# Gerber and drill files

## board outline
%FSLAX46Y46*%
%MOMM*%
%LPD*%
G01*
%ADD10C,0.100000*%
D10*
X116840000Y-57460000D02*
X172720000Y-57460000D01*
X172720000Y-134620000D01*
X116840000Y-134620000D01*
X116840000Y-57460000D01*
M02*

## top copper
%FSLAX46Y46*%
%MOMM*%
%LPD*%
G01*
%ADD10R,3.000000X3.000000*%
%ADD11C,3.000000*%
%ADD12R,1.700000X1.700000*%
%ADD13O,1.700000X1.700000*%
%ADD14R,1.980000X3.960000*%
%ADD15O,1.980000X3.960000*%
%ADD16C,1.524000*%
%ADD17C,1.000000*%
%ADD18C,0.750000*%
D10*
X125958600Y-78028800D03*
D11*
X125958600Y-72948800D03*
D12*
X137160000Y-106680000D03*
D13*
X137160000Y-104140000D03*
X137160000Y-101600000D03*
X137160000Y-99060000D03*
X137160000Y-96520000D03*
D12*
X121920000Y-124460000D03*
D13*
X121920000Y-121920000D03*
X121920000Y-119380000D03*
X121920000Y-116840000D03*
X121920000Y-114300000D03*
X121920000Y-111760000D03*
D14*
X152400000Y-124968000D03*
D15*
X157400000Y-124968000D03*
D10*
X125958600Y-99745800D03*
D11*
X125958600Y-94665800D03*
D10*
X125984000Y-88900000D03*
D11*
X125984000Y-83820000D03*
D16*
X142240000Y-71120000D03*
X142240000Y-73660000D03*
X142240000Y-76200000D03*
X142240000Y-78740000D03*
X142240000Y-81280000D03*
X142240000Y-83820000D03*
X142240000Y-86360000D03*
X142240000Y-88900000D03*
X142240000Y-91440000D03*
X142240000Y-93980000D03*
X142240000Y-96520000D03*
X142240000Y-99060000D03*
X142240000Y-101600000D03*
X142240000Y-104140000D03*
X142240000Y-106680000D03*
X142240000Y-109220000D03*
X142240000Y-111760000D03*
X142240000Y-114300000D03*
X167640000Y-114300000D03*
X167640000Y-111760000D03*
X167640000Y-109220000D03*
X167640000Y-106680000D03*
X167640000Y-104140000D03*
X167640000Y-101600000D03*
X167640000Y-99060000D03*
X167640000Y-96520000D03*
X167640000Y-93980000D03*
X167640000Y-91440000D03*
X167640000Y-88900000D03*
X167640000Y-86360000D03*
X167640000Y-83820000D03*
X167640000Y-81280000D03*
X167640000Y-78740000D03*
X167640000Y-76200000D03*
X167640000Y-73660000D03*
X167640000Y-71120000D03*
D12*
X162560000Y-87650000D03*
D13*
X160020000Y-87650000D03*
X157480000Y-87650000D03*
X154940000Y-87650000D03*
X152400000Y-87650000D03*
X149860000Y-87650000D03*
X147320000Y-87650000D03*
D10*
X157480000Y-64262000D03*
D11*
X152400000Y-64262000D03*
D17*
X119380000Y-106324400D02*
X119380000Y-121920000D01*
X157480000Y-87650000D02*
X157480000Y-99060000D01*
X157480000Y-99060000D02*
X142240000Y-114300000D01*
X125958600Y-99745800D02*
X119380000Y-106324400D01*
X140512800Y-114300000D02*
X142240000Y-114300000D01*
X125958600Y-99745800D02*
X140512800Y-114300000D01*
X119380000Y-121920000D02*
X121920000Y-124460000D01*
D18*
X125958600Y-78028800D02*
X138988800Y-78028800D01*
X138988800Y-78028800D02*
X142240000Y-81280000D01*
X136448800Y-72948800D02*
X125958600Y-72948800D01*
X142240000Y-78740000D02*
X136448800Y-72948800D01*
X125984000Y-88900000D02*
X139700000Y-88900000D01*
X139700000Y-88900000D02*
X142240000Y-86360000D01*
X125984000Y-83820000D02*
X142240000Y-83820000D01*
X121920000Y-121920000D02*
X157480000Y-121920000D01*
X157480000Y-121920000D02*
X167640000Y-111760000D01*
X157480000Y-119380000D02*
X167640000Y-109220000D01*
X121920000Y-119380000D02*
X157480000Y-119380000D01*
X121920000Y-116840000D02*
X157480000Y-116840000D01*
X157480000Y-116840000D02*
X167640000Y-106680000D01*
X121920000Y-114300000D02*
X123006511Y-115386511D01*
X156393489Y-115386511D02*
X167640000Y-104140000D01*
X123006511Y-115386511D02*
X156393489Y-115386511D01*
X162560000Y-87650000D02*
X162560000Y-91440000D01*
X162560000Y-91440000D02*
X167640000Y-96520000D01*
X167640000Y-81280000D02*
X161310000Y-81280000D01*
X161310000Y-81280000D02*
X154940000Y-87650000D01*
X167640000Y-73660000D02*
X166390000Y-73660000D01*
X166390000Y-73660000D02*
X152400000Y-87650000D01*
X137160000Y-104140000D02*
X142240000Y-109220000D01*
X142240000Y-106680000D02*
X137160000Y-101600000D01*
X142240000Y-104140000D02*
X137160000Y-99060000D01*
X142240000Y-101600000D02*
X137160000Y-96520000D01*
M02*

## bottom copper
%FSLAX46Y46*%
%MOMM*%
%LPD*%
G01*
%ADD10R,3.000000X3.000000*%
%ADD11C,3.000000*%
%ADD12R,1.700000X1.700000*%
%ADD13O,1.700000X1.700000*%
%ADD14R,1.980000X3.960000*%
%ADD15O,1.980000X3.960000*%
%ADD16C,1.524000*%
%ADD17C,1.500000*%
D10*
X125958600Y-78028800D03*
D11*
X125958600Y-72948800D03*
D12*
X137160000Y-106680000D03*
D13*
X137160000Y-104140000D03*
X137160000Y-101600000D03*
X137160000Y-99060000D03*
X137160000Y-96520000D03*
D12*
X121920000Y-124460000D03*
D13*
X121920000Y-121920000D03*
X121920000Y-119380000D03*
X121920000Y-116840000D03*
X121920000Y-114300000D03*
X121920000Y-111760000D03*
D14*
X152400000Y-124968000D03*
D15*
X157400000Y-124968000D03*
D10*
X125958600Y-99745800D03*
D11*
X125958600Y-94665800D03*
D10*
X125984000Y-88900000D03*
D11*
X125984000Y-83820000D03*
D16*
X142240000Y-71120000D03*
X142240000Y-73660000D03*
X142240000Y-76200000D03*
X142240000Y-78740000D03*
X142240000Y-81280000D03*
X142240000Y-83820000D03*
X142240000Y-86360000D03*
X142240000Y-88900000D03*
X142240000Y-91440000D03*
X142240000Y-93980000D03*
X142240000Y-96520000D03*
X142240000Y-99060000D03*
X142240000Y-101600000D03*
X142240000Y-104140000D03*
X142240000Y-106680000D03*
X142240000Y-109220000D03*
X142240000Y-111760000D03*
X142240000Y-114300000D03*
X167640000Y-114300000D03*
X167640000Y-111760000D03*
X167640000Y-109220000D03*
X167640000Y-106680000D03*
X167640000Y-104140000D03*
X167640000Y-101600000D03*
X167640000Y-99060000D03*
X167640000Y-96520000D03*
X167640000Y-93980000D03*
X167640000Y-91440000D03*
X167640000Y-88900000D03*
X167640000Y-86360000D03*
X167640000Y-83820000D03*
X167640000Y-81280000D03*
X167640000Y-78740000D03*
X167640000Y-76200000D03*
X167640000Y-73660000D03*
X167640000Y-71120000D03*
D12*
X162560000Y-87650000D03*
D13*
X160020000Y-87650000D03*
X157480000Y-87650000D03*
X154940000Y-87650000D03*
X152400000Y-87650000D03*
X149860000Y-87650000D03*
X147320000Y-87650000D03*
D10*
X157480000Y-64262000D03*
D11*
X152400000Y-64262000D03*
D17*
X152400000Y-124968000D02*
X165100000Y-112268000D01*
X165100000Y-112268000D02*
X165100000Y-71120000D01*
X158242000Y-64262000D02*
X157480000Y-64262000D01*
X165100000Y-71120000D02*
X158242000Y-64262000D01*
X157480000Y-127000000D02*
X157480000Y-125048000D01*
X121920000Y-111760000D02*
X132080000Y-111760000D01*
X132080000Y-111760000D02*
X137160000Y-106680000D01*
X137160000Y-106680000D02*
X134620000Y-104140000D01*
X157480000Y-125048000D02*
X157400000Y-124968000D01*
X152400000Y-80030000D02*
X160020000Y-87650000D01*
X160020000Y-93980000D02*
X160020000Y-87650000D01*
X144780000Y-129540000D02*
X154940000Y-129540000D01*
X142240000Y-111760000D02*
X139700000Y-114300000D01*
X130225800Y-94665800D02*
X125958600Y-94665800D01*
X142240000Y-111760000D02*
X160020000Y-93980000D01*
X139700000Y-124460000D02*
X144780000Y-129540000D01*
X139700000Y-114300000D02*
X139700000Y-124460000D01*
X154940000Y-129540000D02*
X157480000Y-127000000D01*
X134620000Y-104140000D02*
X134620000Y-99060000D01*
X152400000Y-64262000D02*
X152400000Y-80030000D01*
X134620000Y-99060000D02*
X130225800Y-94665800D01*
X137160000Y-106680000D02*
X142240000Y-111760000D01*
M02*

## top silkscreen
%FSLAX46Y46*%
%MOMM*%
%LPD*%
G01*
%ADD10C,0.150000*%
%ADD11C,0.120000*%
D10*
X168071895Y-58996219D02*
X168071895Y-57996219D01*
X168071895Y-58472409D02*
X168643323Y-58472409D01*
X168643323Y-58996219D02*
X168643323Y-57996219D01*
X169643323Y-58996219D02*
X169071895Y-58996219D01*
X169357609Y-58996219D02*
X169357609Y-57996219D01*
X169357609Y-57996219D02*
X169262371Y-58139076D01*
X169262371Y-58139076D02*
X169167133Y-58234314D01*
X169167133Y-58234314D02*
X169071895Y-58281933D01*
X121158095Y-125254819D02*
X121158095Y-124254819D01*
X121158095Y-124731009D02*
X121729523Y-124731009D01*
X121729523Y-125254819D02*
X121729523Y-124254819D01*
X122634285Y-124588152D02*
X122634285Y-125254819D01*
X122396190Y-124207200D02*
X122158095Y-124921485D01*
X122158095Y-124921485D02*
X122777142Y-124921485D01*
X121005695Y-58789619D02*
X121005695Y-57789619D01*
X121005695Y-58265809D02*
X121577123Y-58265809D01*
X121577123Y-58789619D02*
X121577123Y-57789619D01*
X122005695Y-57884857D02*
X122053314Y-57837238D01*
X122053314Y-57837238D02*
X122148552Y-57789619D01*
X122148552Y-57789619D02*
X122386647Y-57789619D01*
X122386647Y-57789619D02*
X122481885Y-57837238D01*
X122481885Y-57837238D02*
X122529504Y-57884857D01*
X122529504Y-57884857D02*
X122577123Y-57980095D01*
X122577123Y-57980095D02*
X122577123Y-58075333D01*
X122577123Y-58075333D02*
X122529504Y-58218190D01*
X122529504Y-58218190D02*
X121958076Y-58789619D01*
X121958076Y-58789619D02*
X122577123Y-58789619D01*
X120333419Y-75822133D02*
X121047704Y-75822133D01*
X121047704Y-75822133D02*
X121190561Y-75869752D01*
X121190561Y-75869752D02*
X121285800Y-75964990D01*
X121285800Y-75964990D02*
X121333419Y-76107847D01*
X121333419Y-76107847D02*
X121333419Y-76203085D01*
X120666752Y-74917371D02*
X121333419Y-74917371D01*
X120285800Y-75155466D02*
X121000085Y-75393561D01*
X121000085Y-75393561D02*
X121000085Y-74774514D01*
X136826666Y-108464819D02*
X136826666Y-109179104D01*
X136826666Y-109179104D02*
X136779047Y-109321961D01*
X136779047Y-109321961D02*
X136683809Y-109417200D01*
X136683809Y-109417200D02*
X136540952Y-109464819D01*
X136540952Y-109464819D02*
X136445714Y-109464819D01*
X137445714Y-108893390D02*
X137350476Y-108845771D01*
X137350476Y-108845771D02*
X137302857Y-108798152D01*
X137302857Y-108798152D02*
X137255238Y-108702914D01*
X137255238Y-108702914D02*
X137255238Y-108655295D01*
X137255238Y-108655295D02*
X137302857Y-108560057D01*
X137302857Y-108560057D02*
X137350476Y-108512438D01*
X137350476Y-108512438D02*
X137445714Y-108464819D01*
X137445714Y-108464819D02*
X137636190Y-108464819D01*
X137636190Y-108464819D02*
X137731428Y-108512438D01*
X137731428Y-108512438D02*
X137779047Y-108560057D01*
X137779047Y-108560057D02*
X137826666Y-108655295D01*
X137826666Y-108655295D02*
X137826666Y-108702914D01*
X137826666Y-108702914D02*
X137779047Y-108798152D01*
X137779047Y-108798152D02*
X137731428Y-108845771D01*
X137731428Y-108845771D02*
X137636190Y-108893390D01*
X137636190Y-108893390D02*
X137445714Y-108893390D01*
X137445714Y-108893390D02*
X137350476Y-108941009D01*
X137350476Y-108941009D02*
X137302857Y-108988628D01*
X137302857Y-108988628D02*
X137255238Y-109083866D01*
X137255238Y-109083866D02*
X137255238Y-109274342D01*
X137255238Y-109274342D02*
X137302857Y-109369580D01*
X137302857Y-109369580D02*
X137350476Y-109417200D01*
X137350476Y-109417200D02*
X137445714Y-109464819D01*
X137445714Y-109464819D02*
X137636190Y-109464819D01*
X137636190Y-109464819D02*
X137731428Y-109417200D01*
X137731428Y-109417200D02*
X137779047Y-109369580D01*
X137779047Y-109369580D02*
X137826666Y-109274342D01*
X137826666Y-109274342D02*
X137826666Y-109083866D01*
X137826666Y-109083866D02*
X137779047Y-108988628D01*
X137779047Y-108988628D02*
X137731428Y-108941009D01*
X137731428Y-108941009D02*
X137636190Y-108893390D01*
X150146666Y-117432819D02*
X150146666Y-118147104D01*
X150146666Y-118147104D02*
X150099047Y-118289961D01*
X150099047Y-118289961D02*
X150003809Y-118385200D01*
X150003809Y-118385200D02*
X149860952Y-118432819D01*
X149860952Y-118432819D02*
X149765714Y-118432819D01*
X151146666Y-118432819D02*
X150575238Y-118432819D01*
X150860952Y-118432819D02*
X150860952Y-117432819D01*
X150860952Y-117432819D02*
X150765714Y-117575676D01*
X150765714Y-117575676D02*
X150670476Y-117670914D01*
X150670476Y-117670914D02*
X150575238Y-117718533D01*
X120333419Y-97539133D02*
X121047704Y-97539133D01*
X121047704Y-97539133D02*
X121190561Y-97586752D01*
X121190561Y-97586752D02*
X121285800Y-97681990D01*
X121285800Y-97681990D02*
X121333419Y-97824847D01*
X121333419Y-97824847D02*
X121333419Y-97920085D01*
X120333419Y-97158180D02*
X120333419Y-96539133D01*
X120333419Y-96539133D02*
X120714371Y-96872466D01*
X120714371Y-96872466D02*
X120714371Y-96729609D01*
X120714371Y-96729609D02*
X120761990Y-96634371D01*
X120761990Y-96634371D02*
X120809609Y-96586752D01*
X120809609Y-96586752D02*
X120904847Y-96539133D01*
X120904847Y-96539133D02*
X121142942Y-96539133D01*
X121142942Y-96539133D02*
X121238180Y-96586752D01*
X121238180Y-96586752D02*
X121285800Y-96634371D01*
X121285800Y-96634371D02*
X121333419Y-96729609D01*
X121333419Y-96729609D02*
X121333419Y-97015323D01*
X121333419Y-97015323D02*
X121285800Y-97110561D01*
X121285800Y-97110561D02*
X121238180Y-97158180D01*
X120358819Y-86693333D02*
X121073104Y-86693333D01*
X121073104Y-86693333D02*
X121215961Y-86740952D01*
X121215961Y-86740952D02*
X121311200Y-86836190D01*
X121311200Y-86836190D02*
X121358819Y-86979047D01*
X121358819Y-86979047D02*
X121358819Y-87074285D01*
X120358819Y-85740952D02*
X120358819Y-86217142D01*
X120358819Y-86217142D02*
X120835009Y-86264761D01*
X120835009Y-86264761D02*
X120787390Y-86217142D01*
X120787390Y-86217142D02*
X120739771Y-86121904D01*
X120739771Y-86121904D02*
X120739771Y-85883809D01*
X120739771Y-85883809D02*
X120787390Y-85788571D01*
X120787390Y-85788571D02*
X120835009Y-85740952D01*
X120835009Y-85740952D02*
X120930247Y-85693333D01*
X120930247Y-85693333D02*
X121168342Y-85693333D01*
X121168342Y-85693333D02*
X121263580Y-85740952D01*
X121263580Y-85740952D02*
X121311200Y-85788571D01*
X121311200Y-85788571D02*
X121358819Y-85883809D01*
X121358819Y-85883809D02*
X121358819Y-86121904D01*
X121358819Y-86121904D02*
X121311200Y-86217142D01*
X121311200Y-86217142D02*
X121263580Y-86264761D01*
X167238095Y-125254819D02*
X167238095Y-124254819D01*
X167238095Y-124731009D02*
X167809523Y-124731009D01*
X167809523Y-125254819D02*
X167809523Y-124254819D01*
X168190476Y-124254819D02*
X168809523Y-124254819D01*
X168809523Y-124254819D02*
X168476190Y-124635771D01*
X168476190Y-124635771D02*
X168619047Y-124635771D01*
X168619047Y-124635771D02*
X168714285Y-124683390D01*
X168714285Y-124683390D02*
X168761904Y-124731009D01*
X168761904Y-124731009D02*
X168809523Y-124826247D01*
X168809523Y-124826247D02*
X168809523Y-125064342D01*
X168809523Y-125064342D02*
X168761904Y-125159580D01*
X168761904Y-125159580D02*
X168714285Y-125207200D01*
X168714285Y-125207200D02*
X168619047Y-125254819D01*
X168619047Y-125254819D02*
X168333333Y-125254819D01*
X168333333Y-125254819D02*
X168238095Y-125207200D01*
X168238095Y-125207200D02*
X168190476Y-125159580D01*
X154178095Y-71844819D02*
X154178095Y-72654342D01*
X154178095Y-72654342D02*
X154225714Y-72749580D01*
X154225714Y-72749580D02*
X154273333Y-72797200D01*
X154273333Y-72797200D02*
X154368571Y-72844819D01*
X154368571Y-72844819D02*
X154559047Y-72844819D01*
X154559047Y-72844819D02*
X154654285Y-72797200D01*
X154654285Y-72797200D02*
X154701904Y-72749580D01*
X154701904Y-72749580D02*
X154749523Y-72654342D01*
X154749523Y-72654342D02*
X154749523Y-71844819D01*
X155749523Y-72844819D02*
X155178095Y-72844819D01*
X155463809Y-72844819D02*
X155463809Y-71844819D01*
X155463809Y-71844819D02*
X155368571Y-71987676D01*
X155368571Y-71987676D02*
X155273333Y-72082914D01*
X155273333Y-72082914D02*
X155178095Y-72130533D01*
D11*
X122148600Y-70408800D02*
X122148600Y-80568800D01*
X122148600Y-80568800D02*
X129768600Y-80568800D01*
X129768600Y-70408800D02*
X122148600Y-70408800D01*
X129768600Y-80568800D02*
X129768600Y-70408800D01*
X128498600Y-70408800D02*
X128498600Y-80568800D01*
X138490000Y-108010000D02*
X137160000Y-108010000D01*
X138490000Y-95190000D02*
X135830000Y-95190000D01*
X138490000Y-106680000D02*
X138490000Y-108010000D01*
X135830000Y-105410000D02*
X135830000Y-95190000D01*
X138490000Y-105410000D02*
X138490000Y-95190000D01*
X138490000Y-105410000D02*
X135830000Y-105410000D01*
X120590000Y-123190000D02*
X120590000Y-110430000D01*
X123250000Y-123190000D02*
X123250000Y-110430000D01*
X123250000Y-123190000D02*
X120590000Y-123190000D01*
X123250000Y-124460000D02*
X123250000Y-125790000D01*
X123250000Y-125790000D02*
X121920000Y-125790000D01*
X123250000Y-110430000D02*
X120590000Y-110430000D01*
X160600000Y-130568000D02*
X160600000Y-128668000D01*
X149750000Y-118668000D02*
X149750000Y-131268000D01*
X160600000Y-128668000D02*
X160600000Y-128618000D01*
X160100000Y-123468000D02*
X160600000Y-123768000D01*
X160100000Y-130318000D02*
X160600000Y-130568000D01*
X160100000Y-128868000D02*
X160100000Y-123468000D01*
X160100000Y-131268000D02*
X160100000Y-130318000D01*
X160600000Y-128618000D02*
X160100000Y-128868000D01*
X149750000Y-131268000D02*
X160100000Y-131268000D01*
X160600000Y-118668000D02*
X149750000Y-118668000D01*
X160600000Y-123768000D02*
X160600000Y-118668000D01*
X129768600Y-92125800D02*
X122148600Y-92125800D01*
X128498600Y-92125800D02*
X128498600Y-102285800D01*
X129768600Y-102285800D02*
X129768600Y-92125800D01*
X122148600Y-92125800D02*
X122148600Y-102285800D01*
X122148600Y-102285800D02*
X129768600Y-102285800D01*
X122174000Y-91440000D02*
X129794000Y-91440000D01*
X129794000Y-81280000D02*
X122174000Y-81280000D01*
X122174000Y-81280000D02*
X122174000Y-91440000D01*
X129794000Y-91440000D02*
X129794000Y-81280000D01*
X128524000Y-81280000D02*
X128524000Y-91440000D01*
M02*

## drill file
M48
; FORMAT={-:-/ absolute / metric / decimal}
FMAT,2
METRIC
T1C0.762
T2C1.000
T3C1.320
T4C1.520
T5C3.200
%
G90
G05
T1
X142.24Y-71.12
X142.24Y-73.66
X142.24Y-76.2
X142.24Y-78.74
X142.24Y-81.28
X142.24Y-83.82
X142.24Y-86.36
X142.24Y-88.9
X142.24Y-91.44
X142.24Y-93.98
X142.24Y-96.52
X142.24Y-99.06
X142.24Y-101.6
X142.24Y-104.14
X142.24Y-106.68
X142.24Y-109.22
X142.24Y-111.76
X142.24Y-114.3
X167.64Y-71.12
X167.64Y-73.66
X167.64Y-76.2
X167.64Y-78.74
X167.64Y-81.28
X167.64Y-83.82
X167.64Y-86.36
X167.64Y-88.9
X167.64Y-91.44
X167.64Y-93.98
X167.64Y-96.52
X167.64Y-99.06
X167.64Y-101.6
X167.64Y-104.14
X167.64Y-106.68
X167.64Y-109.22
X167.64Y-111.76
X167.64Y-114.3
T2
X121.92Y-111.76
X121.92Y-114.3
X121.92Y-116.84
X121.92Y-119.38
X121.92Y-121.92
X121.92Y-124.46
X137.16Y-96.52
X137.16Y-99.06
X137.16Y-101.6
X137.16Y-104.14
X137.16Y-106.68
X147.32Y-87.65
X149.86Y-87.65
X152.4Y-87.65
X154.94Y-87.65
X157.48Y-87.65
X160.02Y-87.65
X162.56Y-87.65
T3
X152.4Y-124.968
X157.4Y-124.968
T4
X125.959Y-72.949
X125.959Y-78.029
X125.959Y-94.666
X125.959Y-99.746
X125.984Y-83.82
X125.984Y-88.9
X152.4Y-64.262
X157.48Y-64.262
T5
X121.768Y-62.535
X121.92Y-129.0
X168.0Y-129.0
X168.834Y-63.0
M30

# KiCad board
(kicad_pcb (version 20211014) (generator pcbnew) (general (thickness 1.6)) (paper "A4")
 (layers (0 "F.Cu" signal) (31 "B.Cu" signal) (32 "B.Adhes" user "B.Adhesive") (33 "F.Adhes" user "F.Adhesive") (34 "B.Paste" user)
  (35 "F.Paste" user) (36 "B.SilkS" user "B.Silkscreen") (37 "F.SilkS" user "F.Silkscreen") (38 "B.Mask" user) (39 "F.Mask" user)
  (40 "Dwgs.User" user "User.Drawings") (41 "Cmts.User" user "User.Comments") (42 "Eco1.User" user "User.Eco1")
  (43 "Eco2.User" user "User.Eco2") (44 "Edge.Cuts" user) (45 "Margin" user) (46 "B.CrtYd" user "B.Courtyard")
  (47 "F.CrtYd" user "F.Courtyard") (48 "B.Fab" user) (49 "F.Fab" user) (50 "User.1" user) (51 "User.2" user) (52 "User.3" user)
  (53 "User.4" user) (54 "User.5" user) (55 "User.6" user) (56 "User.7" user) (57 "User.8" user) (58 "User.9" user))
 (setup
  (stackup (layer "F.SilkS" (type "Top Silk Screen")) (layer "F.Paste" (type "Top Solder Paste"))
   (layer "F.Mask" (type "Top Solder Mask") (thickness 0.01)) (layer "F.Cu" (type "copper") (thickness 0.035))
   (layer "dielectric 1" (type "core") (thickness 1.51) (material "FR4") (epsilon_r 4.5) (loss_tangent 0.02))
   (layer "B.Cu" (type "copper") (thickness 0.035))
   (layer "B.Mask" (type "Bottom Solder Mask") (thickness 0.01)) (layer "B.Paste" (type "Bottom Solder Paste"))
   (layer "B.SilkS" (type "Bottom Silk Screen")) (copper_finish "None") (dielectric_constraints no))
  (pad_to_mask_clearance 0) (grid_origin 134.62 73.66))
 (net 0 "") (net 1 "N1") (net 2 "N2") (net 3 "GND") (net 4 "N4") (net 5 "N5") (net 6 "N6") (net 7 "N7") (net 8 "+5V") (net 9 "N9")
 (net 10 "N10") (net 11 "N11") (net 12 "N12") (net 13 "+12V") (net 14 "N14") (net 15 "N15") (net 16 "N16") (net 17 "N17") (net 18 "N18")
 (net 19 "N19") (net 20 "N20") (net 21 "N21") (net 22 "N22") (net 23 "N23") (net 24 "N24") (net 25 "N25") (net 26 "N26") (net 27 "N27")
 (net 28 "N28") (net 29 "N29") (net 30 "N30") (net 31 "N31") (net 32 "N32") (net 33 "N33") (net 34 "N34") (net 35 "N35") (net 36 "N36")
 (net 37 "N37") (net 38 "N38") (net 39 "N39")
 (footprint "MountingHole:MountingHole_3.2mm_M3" (layer "F.Cu") (at 168.8338 63)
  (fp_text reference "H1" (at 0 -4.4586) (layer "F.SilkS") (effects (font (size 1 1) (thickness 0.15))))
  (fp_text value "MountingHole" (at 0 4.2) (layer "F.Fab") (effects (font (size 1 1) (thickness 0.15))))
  (pad "" np_thru_hole circle (at 0 0) (size 3.2 3.2) (drill 3.2) (layers *.Cu *.Mask)))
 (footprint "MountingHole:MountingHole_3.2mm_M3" (layer "F.Cu") (at 121.92 129)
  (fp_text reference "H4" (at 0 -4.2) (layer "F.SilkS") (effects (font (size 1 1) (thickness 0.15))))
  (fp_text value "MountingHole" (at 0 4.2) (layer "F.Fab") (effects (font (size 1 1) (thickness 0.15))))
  (pad "" np_thru_hole circle (at 0 0) (size 3.2 3.2) (drill 3.2) (layers *.Cu *.Mask)))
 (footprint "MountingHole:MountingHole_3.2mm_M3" (layer "F.Cu") (at 121.7676 62.5348)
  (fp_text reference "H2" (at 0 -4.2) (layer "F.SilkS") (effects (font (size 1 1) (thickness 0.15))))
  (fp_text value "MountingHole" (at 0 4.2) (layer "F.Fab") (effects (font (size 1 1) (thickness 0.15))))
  (pad "" np_thru_hole circle (at 0 0) (size 3.2 3.2) (drill 3.2) (layers *.Cu *.Mask)))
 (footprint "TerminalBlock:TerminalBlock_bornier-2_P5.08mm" (layer "F.Cu") (at 125.9586 78.0288 90)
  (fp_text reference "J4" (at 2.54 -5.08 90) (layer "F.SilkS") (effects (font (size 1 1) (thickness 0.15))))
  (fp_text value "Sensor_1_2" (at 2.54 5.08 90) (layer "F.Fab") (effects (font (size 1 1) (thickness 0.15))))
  (fp_line (start 7.62 -3.81) (end -2.54 -3.81) (layer "F.SilkS") (width 0.12))
  (fp_line (start -2.54 -3.81) (end -2.54 3.81) (layer "F.SilkS") (width 0.12))
  (fp_line (start 7.62 3.81) (end 7.62 -3.81) (layer "F.SilkS") (width 0.12))
  (fp_line (start -2.54 3.81) (end 7.62 3.81) (layer "F.SilkS") (width 0.12))
  (fp_line (start 7.62 2.54) (end -2.54 2.54) (layer "F.SilkS") (width 0.12))
  (pad "1" thru_hole rect (at 0 0 90) (size 3 3) (drill 1.52) (layers *.Cu *.Mask) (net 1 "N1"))
  (pad "2" thru_hole circle (at 5.08 0 90) (size 3 3) (drill 1.52) (layers *.Cu *.Mask) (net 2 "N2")))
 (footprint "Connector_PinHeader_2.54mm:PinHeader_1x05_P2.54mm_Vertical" (layer "F.Cu") (at 137.16 106.68 180)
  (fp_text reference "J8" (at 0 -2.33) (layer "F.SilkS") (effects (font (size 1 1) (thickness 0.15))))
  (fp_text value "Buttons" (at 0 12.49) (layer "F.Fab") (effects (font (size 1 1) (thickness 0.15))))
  (fp_line (start -1.33 -1.33) (end 0 -1.33) (layer "F.SilkS") (width 0.12))
  (fp_line (start -1.33 11.49) (end 1.33 11.49) (layer "F.SilkS") (width 0.12))
  (fp_line (start -1.33 0) (end -1.33 -1.33) (layer "F.SilkS") (width 0.12))
  (fp_line (start 1.33 1.27) (end 1.33 11.49) (layer "F.SilkS") (width 0.12))
  (fp_line (start -1.33 1.27) (end -1.33 11.49) (layer "F.SilkS") (width 0.12))
  (fp_line (start -1.33 1.27) (end 1.33 1.27) (layer "F.SilkS") (width 0.12))
  (pad "1" thru_hole rect (at 0 0 180) (size 1.7 1.7) (drill 1) (layers *.Cu *.Mask) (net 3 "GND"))
  (pad "2" thru_hole oval (at 0 2.54 180) (size 1.7 1.7) (drill 1) (layers *.Cu *.Mask) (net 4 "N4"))
  (pad "3" thru_hole oval (at 0 5.08 180) (size 1.7 1.7) (drill 1) (layers *.Cu *.Mask) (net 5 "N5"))
  (pad "4" thru_hole oval (at 0 7.62 180) (size 1.7 1.7) (drill 1) (layers *.Cu *.Mask) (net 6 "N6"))
  (pad "5" thru_hole oval (at 0 10.16 180) (size 1.7 1.7) (drill 1) (layers *.Cu *.Mask) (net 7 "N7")))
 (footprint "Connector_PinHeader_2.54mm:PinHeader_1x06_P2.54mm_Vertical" (layer "F.Cu") (at 121.92 124.46 180)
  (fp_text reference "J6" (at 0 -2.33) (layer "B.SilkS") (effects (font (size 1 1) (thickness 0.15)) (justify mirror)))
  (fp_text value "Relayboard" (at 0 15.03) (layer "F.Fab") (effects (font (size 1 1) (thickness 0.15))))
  (fp_line (start 1.33 1.27) (end 1.33 14.03) (layer "F.SilkS") (width 0.12))
  (fp_line (start -1.33 1.27) (end -1.33 14.03) (layer "F.SilkS") (width 0.12))
  (fp_line (start -1.33 1.27) (end 1.33 1.27) (layer "F.SilkS") (width 0.12))
  (fp_line (start -1.33 0) (end -1.33 -1.33) (layer "F.SilkS") (width 0.12))
  (fp_line (start -1.33 -1.33) (end 0 -1.33) (layer "F.SilkS") (width 0.12))
  (fp_line (start -1.33 14.03) (end 1.33 14.03) (layer "F.SilkS") (width 0.12))
  (pad "1" thru_hole rect (at 0 0 180) (size 1.7 1.7) (drill 1) (layers *.Cu *.Mask) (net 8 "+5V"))
  (pad "2" thru_hole oval (at 0 2.54 180) (size 1.7 1.7) (drill 1) (layers *.Cu *.Mask) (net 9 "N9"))
  (pad "3" thru_hole oval (at 0 5.08 180) (size 1.7 1.7) (drill 1) (layers *.Cu *.Mask) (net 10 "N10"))
  (pad "4" thru_hole oval (at 0 7.62 180) (size 1.7 1.7) (drill 1) (layers *.Cu *.Mask) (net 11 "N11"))
  (pad "5" thru_hole oval (at 0 10.16 180) (size 1.7 1.7) (drill 1) (layers *.Cu *.Mask) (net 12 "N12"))
  (pad "6" thru_hole oval (at 0 12.7 180) (size 1.7 1.7) (drill 1) (layers *.Cu *.Mask) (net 3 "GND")))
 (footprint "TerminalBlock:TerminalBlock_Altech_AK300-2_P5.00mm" (layer "F.Cu") (at 152.4 124.968)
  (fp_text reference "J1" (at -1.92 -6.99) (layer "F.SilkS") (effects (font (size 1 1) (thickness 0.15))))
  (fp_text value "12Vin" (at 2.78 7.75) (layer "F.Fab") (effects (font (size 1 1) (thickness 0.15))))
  (fp_line (start 8.2 5.6) (end 8.2 3.7) (layer "F.SilkS") (width 0.12))
  (fp_line (start -2.65 -6.3) (end -2.65 6.3) (layer "F.SilkS") (width 0.12))
  (fp_line (start 8.2 3.7) (end 8.2 3.65) (layer "F.SilkS") (width 0.12))
  (fp_line (start 7.7 -1.5) (end 8.2 -1.2) (layer "F.SilkS") (width 0.12))
  (fp_line (start 7.7 5.35) (end 8.2 5.6) (layer "F.SilkS") (width 0.12))
  (fp_line (start 7.7 3.9) (end 7.7 -1.5) (layer "F.SilkS") (width 0.12))
  (fp_line (start 7.7 6.3) (end 7.7 5.35) (layer "F.SilkS") (width 0.12))
  (fp_line (start 8.2 3.65) (end 7.7 3.9) (layer "F.SilkS") (width 0.12))
  (fp_line (start -2.65 6.3) (end 7.7 6.3) (layer "F.SilkS") (width 0.12))
  (fp_line (start 8.2 -6.3) (end -2.65 -6.3) (layer "F.SilkS") (width 0.12))
  (fp_line (start 8.2 -1.2) (end 8.2 -6.3) (layer "F.SilkS") (width 0.12))
  (pad "1" thru_hole rect (at 0 0) (size 1.98 3.96) (drill 1.32) (layers *.Cu *.Mask) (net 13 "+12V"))
  (pad "2" thru_hole oval (at 5 0) (size 1.98 3.96) (drill 1.32) (layers *.Cu *.Mask) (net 3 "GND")))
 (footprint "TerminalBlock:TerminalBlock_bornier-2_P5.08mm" (layer "F.Cu") (at 125.9586 99.7458 90)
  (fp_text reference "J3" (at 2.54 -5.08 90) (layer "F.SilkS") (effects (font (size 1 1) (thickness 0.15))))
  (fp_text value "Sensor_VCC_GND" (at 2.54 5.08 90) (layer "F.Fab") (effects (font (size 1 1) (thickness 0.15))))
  (fp_line (start 7.62 3.81) (end 7.62 -3.81) (layer "F.SilkS") (width 0.12))
  (fp_line (start 7.62 2.54) (end -2.54 2.54) (layer "F.SilkS") (width 0.12))
  (fp_line (start -2.54 3.81) (end 7.62 3.81) (layer "F.SilkS") (width 0.12))
  (fp_line (start 7.62 -3.81) (end -2.54 -3.81) (layer "F.SilkS") (width 0.12))
  (fp_line (start -2.54 -3.81) (end -2.54 3.81) (layer "F.SilkS") (width 0.12))
  (pad "1" thru_hole rect (at 0 0 90) (size 3 3) (drill 1.52) (layers *.Cu *.Mask) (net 8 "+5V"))
  (pad "2" thru_hole circle (at 5.08 0 90) (size 3 3) (drill 1.52) (layers *.Cu *.Mask) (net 3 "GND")))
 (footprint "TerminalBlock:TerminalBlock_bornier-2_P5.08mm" (layer "F.Cu") (at 125.984 88.9 90)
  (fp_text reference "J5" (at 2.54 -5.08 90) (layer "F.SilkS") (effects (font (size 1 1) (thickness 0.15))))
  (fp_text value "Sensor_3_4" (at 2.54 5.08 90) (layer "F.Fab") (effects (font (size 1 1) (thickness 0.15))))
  (fp_line (start -2.54 -3.81) (end -2.54 3.81) (layer "F.SilkS") (width 0.12))
  (fp_line (start 7.62 3.81) (end 7.62 -3.81) (layer "F.SilkS") (width 0.12))
  (fp_line (start 7.62 -3.81) (end -2.54 -3.81) (layer "F.SilkS") (width 0.12))
  (fp_line (start -2.54 3.81) (end 7.62 3.81) (layer "F.SilkS") (width 0.12))
  (fp_line (start 7.62 2.54) (end -2.54 2.54) (layer "F.SilkS") (width 0.12))
  (pad "1" thru_hole rect (at 0 0 90) (size 3 3) (drill 1.52) (layers *.Cu *.Mask) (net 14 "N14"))
  (pad "2" thru_hole circle (at 5.08 0 90) (size 3 3) (drill 1.52) (layers *.Cu *.Mask) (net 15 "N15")))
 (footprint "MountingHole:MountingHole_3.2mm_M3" (layer "F.Cu") (at 168 129)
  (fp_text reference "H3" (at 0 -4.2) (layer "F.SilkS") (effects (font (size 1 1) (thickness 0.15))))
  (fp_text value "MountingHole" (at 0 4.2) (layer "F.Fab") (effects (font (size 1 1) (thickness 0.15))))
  (pad "" np_thru_hole circle (at 0 0) (size 3.2 3.2) (drill 3.2) (layers *.Cu *.Mask)))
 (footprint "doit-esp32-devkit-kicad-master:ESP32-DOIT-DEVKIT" (layer "F.Cu") (at 154.94 68.58)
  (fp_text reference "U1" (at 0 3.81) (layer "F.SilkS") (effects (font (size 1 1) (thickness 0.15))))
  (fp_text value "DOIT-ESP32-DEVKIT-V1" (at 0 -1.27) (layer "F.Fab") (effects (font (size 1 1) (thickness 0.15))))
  (pad "1" thru_hole circle locked (at -12.7 2.54) (size 1.524 1.524) (drill 0.762) (layers *.Cu *.Mask) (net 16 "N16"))
  (pad "2" thru_hole circle locked (at -12.7 5.08) (size 1.524 1.524) (drill 0.762) (layers *.Cu *.Mask) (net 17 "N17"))
  (pad "3" thru_hole circle locked (at -12.7 7.62) (size 1.524 1.524) (drill 0.762) (layers *.Cu *.Mask) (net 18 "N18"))
  (pad "4" thru_hole circle locked (at -12.7 10.16) (size 1.524 1.524) (drill 0.762) (layers *.Cu *.Mask) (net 2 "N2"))
  (pad "5" thru_hole circle locked (at -12.7 12.7) (size 1.524 1.524) (drill 0.762) (layers *.Cu *.Mask) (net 1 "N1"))
  (pad "6" thru_hole circle locked (at -12.7 15.24) (size 1.524 1.524) (drill 0.762) (layers *.Cu *.Mask) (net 15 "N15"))
  (pad "7" thru_hole circle locked (at -12.7 17.78) (size 1.524 1.524) (drill 0.762) (layers *.Cu *.Mask) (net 14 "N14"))
  (pad "8" thru_hole circle locked (at -12.7 20.32) (size 1.524 1.524) (drill 0.762) (layers *.Cu *.Mask) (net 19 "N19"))
  (pad "9" thru_hole circle locked (at -12.7 22.86) (size 1.524 1.524) (drill 0.762) (layers *.Cu *.Mask) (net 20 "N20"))
  (pad "10" thru_hole circle locked (at -12.7 25.4) (size 1.524 1.524) (drill 0.762) (layers *.Cu *.Mask) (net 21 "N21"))
  (pad "11" thru_hole circle locked (at -12.7 27.94) (size 1.524 1.524) (drill 0.762) (layers *.Cu *.Mask) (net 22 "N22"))
  (pad "12" thru_hole circle locked (at -12.7 30.48) (size 1.524 1.524) (drill 0.762) (layers *.Cu *.Mask) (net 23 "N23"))
  (pad "13" thru_hole circle locked (at -12.7 33.02) (size 1.524 1.524) (drill 0.762) (layers *.Cu *.Mask) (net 7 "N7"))
  (pad "14" thru_hole circle locked (at -12.7 35.56) (size 1.524 1.524) (drill 0.762) (layers *.Cu *.Mask) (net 6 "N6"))
  (pad "15" thru_hole circle locked (at -12.7 38.1) (size 1.524 1.524) (drill 0.762) (layers *.Cu *.Mask) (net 5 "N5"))
  (pad "16" thru_hole circle locked (at -12.7 40.64) (size 1.524 1.524) (drill 0.762) (layers *.Cu *.Mask) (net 4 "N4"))
  (pad "17" thru_hole circle locked (at -12.7 43.18) (size 1.524 1.524) (drill 0.762) (layers *.Cu *.Mask) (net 3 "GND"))
  (pad "18" thru_hole circle locked (at -12.7 45.72) (size 1.524 1.524) (drill 0.762) (layers *.Cu *.Mask) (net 8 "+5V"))
  (pad "19" thru_hole circle locked (at 12.7 45.72) (size 1.524 1.524) (drill 0.762) (layers *.Cu *.Mask) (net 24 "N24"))
  (pad "20" thru_hole circle locked (at 12.7 43.18) (size 1.524 1.524) (drill 0.762) (layers *.Cu *.Mask) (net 9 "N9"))
  (pad "21" thru_hole circle locked (at 12.7 40.64) (size 1.524 1.524) (drill 0.762) (layers *.Cu *.Mask) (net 10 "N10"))
  (pad "22" thru_hole circle locked (at 12.7 38.1) (size 1.524 1.524) (drill 0.762) (layers *.Cu *.Mask) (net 11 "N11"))
  (pad "23" thru_hole circle locked (at 12.7 35.56) (size 1.524 1.524) (drill 0.762) (layers *.Cu *.Mask) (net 12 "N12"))
  (pad "24" thru_hole circle locked (at 12.7 33.02) (size 1.524 1.524) (drill 0.762) (layers *.Cu *.Mask) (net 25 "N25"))
  (pad "25" thru_hole circle locked (at 12.7 30.48) (size 1.524 1.524) (drill 0.762) (layers *.Cu *.Mask) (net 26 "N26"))
  (pad "26" thru_hole circle locked (at 12.7 27.94) (size 1.524 1.524) (drill 0.762) (layers *.Cu *.Mask) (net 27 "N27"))
  (pad "27" thru_hole circle locked (at 12.7 25.4) (size 1.524 1.524) (drill 0.762) (layers *.Cu *.Mask) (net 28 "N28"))
  (pad "28" thru_hole circle locked (at 12.7 22.86) (size 1.524 1.524) (drill 0.762) (layers *.Cu *.Mask) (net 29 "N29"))
  (pad "29" thru_hole circle locked (at 12.7 20.32) (size 1.524 1.524) (drill 0.762) (layers *.Cu *.Mask) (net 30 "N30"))
  (pad "30" thru_hole circle locked (at 12.7 17.78) (size 1.524 1.524) (drill 0.762) (layers *.Cu *.Mask) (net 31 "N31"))
  (pad "31" thru_hole circle locked (at 12.7 15.24) (size 1.524 1.524) (drill 0.762) (layers *.Cu *.Mask) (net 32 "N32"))
  (pad "32" thru_hole circle locked (at 12.7 12.7) (size 1.524 1.524) (drill 0.762) (layers *.Cu *.Mask) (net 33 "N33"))
  (pad "33" thru_hole circle locked (at 12.7 10.16) (size 1.524 1.524) (drill 0.762) (layers *.Cu *.Mask) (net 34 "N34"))
  (pad "34" thru_hole circle locked (at 12.7 7.62) (size 1.524 1.524) (drill 0.762) (layers *.Cu *.Mask) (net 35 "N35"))
  (pad "35" thru_hole circle locked (at 12.7 5.08) (size 1.524 1.524) (drill 0.762) (layers *.Cu *.Mask) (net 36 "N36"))
  (pad "36" thru_hole circle locked (at 12.7 2.54) (size 1.524 1.524) (drill 0.762) (layers *.Cu *.Mask) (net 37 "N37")))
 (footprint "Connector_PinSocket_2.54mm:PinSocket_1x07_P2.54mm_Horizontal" (layer "B.Cu") (at 162.56 87.65 90)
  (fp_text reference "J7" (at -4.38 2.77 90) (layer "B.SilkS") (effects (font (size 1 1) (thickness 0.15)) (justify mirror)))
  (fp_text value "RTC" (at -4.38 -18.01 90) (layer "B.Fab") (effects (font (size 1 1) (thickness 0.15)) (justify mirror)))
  (pad "1" thru_hole rect (at 0 0 90) (size 1.7 1.7) (drill 1) (layers *.Cu *.Mask) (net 27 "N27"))
  (pad "2" thru_hole oval (at 0 -2.54 90) (size 1.7 1.7) (drill 1) (layers *.Cu *.Mask) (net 3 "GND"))
  (pad "3" thru_hole oval (at 0 -5.08 90) (size 1.7 1.7) (drill 1) (layers *.Cu *.Mask) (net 8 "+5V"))
  (pad "4" thru_hole oval (at 0 -7.62 90) (size 1.7 1.7) (drill 1) (layers *.Cu *.Mask) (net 33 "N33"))
  (pad "5" thru_hole oval (at 0 -10.16 90) (size 1.7 1.7) (drill 1) (layers *.Cu *.Mask) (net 36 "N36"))
  (pad "6" thru_hole oval (at 0 -12.7 90) (size 1.7 1.7) (drill 1) (layers *.Cu *.Mask) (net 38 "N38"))
  (pad "7" thru_hole oval (at 0 -15.24 90) (size 1.7 1.7) (drill 1) (layers *.Cu *.Mask) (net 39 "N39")))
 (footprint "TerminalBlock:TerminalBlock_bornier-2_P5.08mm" (layer "B.Cu") (at 157.48 64.262 180)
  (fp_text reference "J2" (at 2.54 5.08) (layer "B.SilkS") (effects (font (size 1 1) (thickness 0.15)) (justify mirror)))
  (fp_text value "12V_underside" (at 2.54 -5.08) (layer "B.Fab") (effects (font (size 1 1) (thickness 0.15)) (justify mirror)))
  (pad "1" thru_hole rect (at 0 0 180) (size 3 3) (drill 1.52) (layers *.Cu *.Mask) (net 13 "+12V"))
  (pad "2" thru_hole circle (at 5.08 0 180) (size 3 3) (drill 1.52) (layers *.Cu *.Mask) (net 3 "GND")))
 (gr_rect (start 172.72 57.46) (end 116.84 134.62) (layer "Edge.Cuts") (width 0.1) (fill none))
 (segment (start 152.4 124.968) (end 165.1 112.268) (width 1.5) (layer "B.Cu") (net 13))
 (segment (start 165.1 112.268) (end 165.1 71.12) (width 1.5) (layer "B.Cu") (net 13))
 (segment (start 158.242 64.262) (end 157.48 64.262) (width 1.5) (layer "B.Cu") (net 13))
 (segment (start 165.1 71.12) (end 158.242 64.262) (width 1.5) (layer "B.Cu") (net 13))
 (segment (start 157.48 127) (end 157.48 125.048) (width 1.5) (layer "B.Cu") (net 3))
 (segment (start 121.92 111.76) (end 132.08 111.76) (width 1.5) (layer "B.Cu") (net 3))
 (segment (start 132.08 111.76) (end 137.16 106.68) (width 1.5) (layer "B.Cu") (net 3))
 (segment (start 137.16 106.68) (end 134.62 104.14) (width 1.5) (layer "B.Cu") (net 3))
 (segment (start 157.48 125.048) (end 157.4 124.968) (width 1.5) (layer "B.Cu") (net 3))
 (segment (start 152.4 80.03) (end 160.02 87.65) (width 1.5) (layer "B.Cu") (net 3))
 (segment (start 160.02 93.98) (end 160.02 87.65) (width 1.5) (layer "B.Cu") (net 3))
 (segment (start 144.78 129.54) (end 154.94 129.54) (width 1.5) (layer "B.Cu") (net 3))
 (segment (start 142.24 111.76) (end 139.7 114.3) (width 1.5) (layer "B.Cu") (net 3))
 (segment (start 130.2258 94.6658) (end 125.9586 94.6658) (width 1.5) (layer "B.Cu") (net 3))
 (segment (start 142.24 111.76) (end 160.02 93.98) (width 1.5) (layer "B.Cu") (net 3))
 (segment (start 139.7 124.46) (end 144.78 129.54) (width 1.5) (layer "B.Cu") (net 3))
 (segment (start 139.7 114.3) (end 139.7 124.46) (width 1.5) (layer "B.Cu") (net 3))
 (segment (start 154.94 129.54) (end 157.48 127) (width 1.5) (layer "B.Cu") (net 3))
 (segment (start 134.62 104.14) (end 134.62 99.06) (width 1.5) (layer "B.Cu") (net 3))
 (segment (start 152.4 64.262) (end 152.4 80.03) (width 1.5) (layer "B.Cu") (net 3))
 (segment (start 134.62 99.06) (end 130.2258 94.6658) (width 1.5) (layer "B.Cu") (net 3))
 (segment (start 137.16 106.68) (end 142.24 111.76) (width 1.5) (layer "B.Cu") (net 3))
 (segment (start 119.38 106.3244) (end 119.38 121.92) (width 1) (layer "F.Cu") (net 8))
 (segment (start 157.48 87.65) (end 157.48 99.06) (width 1) (layer "F.Cu") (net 8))
 (segment (start 157.48 99.06) (end 142.24 114.3) (width 1) (layer "F.Cu") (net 8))
 (segment (start 125.9586 99.7458) (end 119.38 106.3244) (width 1) (layer "F.Cu") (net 8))
 (segment (start 140.5128 114.3) (end 142.24 114.3) (width 1) (layer "F.Cu") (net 8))
 (segment (start 125.9586 99.7458) (end 140.5128 114.3) (width 1) (layer "F.Cu") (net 8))
 (segment (start 119.38 121.92) (end 121.92 124.46) (width 1) (layer "F.Cu") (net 8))
 (segment (start 125.9586 78.0288) (end 138.9888 78.0288) (width 0.75) (layer "F.Cu") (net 1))
 (segment (start 138.9888 78.0288) (end 142.24 81.28) (width 0.75) (layer "F.Cu") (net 1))
 (segment (start 136.4488 72.9488) (end 125.9586 72.9488) (width 0.75) (layer "F.Cu") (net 2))
 (segment (start 142.24 78.74) (end 136.4488 72.9488) (width 0.75) (layer "F.Cu") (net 2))
 (segment (start 125.984 88.9) (end 139.7 88.9) (width 0.75) (layer "F.Cu") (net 14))
 (segment (start 139.7 88.9) (end 142.24 86.36) (width 0.75) (layer "F.Cu") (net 14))
 (segment (start 125.984 83.82) (end 142.24 83.82) (width 0.75) (layer "F.Cu") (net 15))
 (segment (start 121.92 121.92) (end 157.48 121.92) (width 0.75) (layer "F.Cu") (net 9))
 (segment (start 157.48 121.92) (end 167.64 111.76) (width 0.75) (layer "F.Cu") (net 9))
 (segment (start 157.48 119.38) (end 167.64 109.22) (width 0.75) (layer "F.Cu") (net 10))
 (segment (start 121.92 119.38) (end 157.48 119.38) (width 0.75) (layer "F.Cu") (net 10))
 (segment (start 121.92 116.84) (end 157.48 116.84) (width 0.75) (layer "F.Cu") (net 11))
 (segment (start 157.48 116.84) (end 167.64 106.68) (width 0.75) (layer "F.Cu") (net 11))
 (segment (start 121.92 114.3) (end 123.006511 115.386511) (width 0.75) (layer "F.Cu") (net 12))
 (segment (start 156.393489 115.386511) (end 167.64 104.14) (width 0.75) (layer "F.Cu") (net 12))
 (segment (start 123.006511 115.386511) (end 156.393489 115.386511) (width 0.75) (layer "F.Cu") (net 12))
 (segment (start 162.56 87.65) (end 162.56 91.44) (width 0.75) (layer "F.Cu") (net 27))
 (segment (start 162.56 91.44) (end 167.64 96.52) (width 0.75) (layer "F.Cu") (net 27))
 (segment (start 167.64 81.28) (end 161.31 81.28) (width 0.75) (layer "F.Cu") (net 33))
 (segment (start 161.31 81.28) (end 154.94 87.65) (width 0.75) (layer "F.Cu") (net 33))
 (segment (start 167.64 73.66) (end 166.39 73.66) (width 0.75) (layer "F.Cu") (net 36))
 (segment (start 166.39 73.66) (end 152.4 87.65) (width 0.75) (layer "F.Cu") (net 36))
 (segment (start 137.16 104.14) (end 142.24 109.22) (width 0.75) (layer "F.Cu") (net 4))
 (segment (start 142.24 106.68) (end 137.16 101.6) (width 0.75) (layer "F.Cu") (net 5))
 (segment (start 142.24 104.14) (end 137.16 99.06) (width 0.75) (layer "F.Cu") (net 6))
 (segment (start 142.24 101.6) (end 137.16 96.52) (width 0.75) (layer "F.Cu") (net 7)))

